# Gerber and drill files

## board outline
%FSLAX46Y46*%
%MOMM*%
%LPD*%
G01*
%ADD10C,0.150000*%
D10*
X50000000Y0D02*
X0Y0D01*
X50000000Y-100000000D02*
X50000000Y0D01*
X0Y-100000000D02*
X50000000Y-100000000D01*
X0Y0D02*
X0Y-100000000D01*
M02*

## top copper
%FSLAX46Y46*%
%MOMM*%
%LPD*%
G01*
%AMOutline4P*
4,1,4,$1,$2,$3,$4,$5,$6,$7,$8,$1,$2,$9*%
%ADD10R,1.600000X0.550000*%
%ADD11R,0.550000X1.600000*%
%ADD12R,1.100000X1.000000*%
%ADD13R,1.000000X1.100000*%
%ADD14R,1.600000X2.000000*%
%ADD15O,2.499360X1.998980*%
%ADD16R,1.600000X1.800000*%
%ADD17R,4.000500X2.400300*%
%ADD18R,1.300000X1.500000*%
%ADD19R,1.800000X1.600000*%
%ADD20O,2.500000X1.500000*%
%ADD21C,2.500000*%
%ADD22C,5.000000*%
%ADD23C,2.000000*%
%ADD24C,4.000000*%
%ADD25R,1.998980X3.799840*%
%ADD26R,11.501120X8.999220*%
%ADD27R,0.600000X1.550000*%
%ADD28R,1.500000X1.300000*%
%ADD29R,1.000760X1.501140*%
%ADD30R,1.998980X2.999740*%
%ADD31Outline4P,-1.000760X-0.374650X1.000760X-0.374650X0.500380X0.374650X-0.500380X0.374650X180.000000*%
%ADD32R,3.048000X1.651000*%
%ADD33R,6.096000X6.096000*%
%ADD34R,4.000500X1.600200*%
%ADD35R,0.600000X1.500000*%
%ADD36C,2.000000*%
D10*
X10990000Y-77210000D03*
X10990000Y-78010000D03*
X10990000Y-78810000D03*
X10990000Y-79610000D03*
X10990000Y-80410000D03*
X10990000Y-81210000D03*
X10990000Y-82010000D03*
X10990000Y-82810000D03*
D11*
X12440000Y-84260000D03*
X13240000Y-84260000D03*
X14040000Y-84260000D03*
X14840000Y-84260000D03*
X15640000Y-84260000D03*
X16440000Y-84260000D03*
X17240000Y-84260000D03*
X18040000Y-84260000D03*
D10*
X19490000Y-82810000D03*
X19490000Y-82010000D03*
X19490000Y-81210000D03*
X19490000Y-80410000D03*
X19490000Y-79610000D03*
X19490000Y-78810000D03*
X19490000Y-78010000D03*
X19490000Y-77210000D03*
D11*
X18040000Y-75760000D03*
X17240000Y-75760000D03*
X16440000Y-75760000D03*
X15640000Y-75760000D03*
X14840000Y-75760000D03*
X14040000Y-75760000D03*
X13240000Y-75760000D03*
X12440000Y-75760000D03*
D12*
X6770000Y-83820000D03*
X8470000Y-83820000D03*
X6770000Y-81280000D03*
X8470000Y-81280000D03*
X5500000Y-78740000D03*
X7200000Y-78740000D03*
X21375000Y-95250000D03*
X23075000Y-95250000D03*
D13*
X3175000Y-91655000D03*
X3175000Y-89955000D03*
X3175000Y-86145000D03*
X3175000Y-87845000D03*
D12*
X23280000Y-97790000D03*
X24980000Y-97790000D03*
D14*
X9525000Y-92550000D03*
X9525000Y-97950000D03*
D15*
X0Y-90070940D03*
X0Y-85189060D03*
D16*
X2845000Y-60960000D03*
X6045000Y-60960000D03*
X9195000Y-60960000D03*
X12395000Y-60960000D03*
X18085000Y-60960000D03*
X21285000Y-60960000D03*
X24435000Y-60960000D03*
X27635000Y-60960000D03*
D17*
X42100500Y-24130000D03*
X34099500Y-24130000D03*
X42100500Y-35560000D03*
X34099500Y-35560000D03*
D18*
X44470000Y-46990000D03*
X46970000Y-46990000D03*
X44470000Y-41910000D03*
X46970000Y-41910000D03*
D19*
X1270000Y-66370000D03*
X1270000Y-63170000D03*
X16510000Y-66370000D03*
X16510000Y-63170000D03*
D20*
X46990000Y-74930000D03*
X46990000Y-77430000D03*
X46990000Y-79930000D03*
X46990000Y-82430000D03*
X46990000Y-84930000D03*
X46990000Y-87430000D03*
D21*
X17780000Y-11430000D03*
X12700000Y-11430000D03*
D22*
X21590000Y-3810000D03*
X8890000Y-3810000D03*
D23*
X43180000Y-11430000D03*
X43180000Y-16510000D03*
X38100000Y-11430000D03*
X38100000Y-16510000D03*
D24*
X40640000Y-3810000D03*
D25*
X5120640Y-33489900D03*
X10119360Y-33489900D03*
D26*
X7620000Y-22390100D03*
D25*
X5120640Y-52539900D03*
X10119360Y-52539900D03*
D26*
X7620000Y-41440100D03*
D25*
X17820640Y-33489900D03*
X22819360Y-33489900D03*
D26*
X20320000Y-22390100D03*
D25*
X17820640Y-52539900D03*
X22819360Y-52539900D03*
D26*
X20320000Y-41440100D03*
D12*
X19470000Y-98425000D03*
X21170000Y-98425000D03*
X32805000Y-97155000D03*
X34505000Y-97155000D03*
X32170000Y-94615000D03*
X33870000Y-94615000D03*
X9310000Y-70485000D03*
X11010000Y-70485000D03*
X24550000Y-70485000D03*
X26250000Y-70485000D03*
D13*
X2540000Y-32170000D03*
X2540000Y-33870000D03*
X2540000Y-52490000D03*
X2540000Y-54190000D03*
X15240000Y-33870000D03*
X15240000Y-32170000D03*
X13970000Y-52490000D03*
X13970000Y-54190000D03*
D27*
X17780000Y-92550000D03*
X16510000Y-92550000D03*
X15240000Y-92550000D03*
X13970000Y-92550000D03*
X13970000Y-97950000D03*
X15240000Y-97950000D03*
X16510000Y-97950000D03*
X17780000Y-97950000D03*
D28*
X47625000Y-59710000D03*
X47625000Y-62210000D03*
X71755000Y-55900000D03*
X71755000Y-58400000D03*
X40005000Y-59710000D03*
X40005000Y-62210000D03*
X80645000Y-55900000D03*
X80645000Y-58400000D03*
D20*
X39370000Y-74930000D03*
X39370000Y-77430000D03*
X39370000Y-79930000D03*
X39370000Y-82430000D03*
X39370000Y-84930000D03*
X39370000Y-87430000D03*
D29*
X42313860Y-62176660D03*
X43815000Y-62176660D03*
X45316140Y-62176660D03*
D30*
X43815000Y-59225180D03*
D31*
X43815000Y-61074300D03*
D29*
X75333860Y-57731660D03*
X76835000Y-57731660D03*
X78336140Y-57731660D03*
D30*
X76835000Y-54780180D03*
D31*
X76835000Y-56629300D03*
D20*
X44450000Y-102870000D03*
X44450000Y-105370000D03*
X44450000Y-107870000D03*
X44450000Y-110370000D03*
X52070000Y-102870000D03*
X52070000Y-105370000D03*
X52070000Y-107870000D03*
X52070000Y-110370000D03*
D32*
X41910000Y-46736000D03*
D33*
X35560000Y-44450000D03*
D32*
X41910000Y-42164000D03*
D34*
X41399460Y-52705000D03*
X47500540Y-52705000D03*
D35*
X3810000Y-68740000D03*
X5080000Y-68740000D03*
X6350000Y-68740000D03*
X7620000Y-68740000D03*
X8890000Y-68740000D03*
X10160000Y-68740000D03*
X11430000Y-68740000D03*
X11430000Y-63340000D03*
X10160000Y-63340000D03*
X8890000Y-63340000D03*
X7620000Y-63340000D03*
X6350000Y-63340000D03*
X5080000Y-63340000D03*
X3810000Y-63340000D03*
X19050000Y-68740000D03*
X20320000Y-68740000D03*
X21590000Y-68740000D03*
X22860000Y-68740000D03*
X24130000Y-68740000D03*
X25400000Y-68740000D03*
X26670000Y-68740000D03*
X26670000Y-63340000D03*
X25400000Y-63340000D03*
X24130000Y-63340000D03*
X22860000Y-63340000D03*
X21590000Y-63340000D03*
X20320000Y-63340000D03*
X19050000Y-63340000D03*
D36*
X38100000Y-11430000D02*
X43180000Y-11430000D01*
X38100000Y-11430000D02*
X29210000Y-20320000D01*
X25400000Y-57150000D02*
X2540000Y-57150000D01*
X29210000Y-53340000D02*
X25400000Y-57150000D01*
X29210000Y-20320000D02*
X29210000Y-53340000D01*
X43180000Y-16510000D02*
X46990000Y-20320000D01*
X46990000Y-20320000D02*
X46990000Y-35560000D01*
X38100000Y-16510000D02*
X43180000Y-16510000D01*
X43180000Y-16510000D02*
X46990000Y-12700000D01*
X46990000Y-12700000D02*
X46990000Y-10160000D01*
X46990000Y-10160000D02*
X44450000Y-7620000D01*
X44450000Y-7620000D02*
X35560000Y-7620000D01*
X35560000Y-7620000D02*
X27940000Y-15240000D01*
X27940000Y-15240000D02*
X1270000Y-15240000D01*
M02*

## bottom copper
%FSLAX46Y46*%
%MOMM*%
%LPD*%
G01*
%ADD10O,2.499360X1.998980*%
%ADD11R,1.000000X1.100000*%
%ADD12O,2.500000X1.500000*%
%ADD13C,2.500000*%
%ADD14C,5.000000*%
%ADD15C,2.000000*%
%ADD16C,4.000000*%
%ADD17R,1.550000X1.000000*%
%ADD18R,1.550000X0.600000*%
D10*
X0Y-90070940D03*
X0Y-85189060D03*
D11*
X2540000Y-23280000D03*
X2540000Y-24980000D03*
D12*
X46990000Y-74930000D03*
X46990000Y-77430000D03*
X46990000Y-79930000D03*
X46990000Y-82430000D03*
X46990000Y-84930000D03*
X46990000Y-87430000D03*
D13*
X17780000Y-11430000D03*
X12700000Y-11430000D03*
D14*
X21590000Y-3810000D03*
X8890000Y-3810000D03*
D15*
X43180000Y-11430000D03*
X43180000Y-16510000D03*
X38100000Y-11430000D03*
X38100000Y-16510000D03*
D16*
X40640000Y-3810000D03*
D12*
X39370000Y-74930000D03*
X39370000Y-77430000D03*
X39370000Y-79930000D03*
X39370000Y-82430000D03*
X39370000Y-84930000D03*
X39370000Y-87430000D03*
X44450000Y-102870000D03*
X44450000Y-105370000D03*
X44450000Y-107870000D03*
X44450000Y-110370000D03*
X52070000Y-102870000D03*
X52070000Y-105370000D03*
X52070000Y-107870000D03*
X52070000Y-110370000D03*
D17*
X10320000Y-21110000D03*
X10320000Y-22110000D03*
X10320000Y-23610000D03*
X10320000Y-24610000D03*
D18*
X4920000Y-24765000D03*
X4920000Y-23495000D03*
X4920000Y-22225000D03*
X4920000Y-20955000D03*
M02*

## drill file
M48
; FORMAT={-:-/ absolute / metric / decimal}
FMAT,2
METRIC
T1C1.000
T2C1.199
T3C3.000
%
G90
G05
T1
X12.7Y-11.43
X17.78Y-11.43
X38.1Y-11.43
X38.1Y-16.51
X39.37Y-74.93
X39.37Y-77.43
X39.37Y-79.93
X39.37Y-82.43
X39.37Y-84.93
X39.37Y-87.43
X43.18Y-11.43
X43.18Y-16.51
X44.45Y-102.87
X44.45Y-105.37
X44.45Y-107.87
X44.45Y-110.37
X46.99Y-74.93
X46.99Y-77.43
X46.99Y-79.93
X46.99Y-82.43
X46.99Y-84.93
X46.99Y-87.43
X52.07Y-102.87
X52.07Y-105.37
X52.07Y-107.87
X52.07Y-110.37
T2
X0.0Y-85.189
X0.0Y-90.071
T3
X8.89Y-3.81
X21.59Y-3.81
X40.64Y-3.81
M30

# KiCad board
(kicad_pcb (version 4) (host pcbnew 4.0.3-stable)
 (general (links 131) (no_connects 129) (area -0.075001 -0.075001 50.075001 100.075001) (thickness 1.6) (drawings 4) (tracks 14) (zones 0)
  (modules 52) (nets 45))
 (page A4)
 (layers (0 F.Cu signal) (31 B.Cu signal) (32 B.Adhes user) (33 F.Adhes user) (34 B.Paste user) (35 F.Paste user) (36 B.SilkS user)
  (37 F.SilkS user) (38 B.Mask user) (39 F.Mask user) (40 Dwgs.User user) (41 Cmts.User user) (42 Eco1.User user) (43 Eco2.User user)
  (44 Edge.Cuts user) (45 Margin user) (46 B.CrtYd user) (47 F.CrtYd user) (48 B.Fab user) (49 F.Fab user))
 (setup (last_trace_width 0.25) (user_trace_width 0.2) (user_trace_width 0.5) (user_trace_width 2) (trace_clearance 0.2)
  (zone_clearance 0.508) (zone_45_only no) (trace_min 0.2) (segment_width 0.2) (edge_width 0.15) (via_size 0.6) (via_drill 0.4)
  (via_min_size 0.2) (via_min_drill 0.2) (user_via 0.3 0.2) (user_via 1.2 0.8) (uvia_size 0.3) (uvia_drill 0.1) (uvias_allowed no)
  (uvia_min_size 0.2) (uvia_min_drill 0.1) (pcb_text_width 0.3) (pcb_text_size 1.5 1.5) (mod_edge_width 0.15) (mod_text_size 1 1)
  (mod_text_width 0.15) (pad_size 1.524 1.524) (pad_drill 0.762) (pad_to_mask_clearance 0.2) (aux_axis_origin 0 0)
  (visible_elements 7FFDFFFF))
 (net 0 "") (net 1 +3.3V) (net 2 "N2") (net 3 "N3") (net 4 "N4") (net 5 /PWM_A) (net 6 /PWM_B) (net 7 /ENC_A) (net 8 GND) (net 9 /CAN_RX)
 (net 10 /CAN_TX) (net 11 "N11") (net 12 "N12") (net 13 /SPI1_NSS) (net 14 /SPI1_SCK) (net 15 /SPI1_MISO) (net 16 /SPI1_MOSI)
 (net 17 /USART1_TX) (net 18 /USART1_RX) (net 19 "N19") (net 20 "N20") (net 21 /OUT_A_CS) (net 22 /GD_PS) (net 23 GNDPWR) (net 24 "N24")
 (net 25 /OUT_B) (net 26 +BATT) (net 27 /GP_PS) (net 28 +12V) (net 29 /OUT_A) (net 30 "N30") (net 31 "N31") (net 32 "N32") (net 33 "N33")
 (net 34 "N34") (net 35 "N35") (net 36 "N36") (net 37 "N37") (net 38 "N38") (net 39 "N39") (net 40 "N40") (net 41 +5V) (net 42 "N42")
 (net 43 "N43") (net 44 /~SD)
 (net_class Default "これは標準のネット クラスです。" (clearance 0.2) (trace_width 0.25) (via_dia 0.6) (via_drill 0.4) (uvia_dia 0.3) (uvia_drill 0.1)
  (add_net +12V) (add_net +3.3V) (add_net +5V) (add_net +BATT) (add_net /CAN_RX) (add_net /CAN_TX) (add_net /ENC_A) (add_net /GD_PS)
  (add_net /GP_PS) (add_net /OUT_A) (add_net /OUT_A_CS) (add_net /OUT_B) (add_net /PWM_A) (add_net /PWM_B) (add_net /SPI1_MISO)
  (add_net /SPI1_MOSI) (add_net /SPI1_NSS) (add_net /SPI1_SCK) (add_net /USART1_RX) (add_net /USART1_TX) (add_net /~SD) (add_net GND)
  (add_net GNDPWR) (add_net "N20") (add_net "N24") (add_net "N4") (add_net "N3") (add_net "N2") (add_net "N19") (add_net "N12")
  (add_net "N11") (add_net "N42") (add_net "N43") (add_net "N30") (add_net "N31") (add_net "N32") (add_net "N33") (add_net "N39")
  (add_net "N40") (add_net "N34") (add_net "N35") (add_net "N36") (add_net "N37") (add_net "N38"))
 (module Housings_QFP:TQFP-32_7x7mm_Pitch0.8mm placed (layer F.Cu) (at 15.24 80.01)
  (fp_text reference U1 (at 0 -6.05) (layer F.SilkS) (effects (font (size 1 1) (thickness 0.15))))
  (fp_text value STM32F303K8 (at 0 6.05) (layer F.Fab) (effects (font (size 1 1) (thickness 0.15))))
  (pad 1 smd rect (at -4.25 -2.8) (size 1.6 0.55) (layers F.Cu F.Paste F.Mask) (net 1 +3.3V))
  (pad 2 smd rect (at -4.25 -2) (size 1.6 0.55) (layers F.Cu F.Paste F.Mask) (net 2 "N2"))
  (pad 3 smd rect (at -4.25 -1.2) (size 1.6 0.55) (layers F.Cu F.Paste F.Mask) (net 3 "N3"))
  (pad 4 smd rect (at -4.25 -0.4) (size 1.6 0.55) (layers F.Cu F.Paste F.Mask) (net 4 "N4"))
  (pad 5 smd rect (at -4.25 0.4) (size 1.6 0.55) (layers F.Cu F.Paste F.Mask) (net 1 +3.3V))
  (pad 6 smd rect (at -4.25 1.2) (size 1.6 0.55) (layers F.Cu F.Paste F.Mask) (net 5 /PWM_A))
  (pad 7 smd rect (at -4.25 2) (size 1.6 0.55) (layers F.Cu F.Paste F.Mask) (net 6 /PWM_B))
  (pad 8 smd rect (at -4.25 2.8) (size 1.6 0.55) (layers F.Cu F.Paste F.Mask))
  (pad 9 smd rect (at -2.8 4.25 90) (size 1.6 0.55) (layers F.Cu F.Paste F.Mask))
  (pad 10 smd rect (at -2 4.25 90) (size 1.6 0.55) (layers F.Cu F.Paste F.Mask))
  (pad 11 smd rect (at -1.2 4.25 90) (size 1.6 0.55) (layers F.Cu F.Paste F.Mask))
  (pad 12 smd rect (at -0.4 4.25 90) (size 1.6 0.55) (layers F.Cu F.Paste F.Mask) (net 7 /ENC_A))
  (pad 13 smd rect (at 0.4 4.25 90) (size 1.6 0.55) (layers F.Cu F.Paste F.Mask))
  (pad 14 smd rect (at 1.2 4.25 90) (size 1.6 0.55) (layers F.Cu F.Paste F.Mask))
  (pad 15 smd rect (at 2 4.25 90) (size 1.6 0.55) (layers F.Cu F.Paste F.Mask))
  (pad 16 smd rect (at 2.8 4.25 90) (size 1.6 0.55) (layers F.Cu F.Paste F.Mask) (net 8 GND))
  (pad 17 smd rect (at 4.25 2.8) (size 1.6 0.55) (layers F.Cu F.Paste F.Mask) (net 1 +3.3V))
  (pad 18 smd rect (at 4.25 2) (size 1.6 0.55) (layers F.Cu F.Paste F.Mask))
  (pad 19 smd rect (at 4.25 1.2) (size 1.6 0.55) (layers F.Cu F.Paste F.Mask))
  (pad 20 smd rect (at 4.25 0.4) (size 1.6 0.55) (layers F.Cu F.Paste F.Mask))
  (pad 21 smd rect (at 4.25 -0.4) (size 1.6 0.55) (layers F.Cu F.Paste F.Mask) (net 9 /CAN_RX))
  (pad 22 smd rect (at 4.25 -1.2) (size 1.6 0.55) (layers F.Cu F.Paste F.Mask) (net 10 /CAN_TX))
  (pad 23 smd rect (at 4.25 -2) (size 1.6 0.55) (layers F.Cu F.Paste F.Mask) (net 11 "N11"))
  (pad 24 smd rect (at 4.25 -2.8) (size 1.6 0.55) (layers F.Cu F.Paste F.Mask) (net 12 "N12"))
  (pad 25 smd rect (at 2.8 -4.25 90) (size 1.6 0.55) (layers F.Cu F.Paste F.Mask) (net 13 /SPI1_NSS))
  (pad 26 smd rect (at 2 -4.25 90) (size 1.6 0.55) (layers F.Cu F.Paste F.Mask) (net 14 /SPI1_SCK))
  (pad 27 smd rect (at 1.2 -4.25 90) (size 1.6 0.55) (layers F.Cu F.Paste F.Mask) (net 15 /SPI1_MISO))
  (pad 28 smd rect (at 0.4 -4.25 90) (size 1.6 0.55) (layers F.Cu F.Paste F.Mask) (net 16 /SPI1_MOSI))
  (pad 29 smd rect (at -0.4 -4.25 90) (size 1.6 0.55) (layers F.Cu F.Paste F.Mask) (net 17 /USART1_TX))
  (pad 30 smd rect (at -1.2 -4.25 90) (size 1.6 0.55) (layers F.Cu F.Paste F.Mask) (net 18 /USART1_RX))
  (pad 31 smd rect (at -2 -4.25 90) (size 1.6 0.55) (layers F.Cu F.Paste F.Mask) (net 8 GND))
  (pad 32 smd rect (at -2.8 -4.25 90) (size 1.6 0.55) (layers F.Cu F.Paste F.Mask) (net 8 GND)))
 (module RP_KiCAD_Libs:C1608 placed (layer F.Cu) (at 7.62 83.82)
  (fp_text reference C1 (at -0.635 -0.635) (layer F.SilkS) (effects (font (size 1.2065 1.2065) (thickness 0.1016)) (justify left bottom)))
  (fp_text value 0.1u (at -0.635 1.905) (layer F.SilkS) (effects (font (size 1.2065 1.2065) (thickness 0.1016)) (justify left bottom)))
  (pad 1 smd rect (at -0.85 0) (size 1.1 1) (layers F.Cu F.Paste F.Mask) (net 1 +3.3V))
  (pad 2 smd rect (at 0.85 0) (size 1.1 1) (layers F.Cu F.Paste F.Mask) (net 8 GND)))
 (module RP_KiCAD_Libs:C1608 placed (layer F.Cu) (at 7.62 81.28)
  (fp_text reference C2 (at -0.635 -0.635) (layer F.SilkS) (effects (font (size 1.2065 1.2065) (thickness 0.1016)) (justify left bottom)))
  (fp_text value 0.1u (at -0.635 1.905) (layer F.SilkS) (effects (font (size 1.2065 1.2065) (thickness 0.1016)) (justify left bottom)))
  (pad 1 smd rect (at -0.85 0) (size 1.1 1) (layers F.Cu F.Paste F.Mask) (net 1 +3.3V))
  (pad 2 smd rect (at 0.85 0) (size 1.1 1) (layers F.Cu F.Paste F.Mask) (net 8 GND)))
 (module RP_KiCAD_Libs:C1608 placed (layer F.Cu) (at 6.35 78.74)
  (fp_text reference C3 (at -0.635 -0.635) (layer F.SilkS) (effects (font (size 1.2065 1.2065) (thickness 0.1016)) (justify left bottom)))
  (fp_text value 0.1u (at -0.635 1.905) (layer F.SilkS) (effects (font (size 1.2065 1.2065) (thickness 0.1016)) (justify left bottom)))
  (pad 1 smd rect (at -0.85 0) (size 1.1 1) (layers F.Cu F.Paste F.Mask) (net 1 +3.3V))
  (pad 2 smd rect (at 0.85 0) (size 1.1 1) (layers F.Cu F.Paste F.Mask) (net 8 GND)))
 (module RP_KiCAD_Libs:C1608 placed (layer F.Cu) (at 22.225 95.25)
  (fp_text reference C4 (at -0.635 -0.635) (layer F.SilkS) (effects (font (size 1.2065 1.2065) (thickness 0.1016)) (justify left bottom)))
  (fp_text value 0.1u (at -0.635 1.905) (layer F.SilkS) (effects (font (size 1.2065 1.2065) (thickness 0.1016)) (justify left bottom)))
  (pad 1 smd rect (at -0.85 0) (size 1.1 1) (layers F.Cu F.Paste F.Mask) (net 8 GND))
  (pad 2 smd rect (at 0.85 0) (size 1.1 1) (layers F.Cu F.Paste F.Mask) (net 4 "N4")))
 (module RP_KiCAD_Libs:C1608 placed (layer F.Cu) (at 3.175 90.805 90)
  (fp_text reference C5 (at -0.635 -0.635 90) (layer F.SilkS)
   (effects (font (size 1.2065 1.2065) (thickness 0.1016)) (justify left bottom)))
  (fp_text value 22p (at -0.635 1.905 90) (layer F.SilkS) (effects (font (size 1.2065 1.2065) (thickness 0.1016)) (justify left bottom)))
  (pad 1 smd rect (at -0.85 0 90) (size 1.1 1) (layers F.Cu F.Paste F.Mask) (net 3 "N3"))
  (pad 2 smd rect (at 0.85 0 90) (size 1.1 1) (layers F.Cu F.Paste F.Mask) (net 8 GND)))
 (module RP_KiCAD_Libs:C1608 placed (layer F.Cu) (at 3.175 86.995 270)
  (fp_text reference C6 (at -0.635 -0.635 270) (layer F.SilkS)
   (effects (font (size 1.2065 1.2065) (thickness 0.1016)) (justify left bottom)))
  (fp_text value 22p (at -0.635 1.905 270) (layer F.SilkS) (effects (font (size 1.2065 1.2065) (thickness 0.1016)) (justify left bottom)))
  (pad 1 smd rect (at -0.85 0 270) (size 1.1 1) (layers F.Cu F.Paste F.Mask) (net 2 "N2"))
  (pad 2 smd rect (at 0.85 0 270) (size 1.1 1) (layers F.Cu F.Paste F.Mask) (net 8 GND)))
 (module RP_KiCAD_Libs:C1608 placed (layer F.Cu) (at 24.13 97.79)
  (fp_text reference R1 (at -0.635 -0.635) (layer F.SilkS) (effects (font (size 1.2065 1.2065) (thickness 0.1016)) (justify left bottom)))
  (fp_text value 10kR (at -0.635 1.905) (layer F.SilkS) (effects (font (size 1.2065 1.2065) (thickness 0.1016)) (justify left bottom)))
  (pad 1 smd rect (at -0.85 0) (size 1.1 1) (layers F.Cu F.Paste F.Mask) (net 4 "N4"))
  (pad 2 smd rect (at 0.85 0) (size 1.1 1) (layers F.Cu F.Paste F.Mask) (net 1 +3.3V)))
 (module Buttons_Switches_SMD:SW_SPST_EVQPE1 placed (layer F.Cu) (at 9.525 95.25 90)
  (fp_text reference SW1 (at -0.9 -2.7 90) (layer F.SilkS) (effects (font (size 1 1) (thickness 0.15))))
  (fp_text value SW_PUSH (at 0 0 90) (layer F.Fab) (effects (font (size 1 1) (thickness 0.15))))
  (pad 2 smd rect (at 2.7 0 90) (size 2 1.6) (layers F.Cu F.Paste F.Mask) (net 4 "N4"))
  (pad 1 smd rect (at -2.7 0 90) (size 2 1.6) (layers F.Cu F.Paste F.Mask) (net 8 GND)))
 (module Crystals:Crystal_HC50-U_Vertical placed (layer F.Cu) (at 0 87.63 90)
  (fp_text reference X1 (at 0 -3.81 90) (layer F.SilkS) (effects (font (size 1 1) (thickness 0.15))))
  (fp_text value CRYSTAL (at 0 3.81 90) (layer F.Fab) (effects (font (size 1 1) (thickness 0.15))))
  (pad 1 thru_hole oval (at -2.44094 0 90) (size 1.99898 2.49936) (drill 1.19888) (layers *.Cu *.Mask F.SilkS) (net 3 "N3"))
  (pad 2 thru_hole oval (at 2.44094 0 90) (size 1.99898 2.49936) (drill 1.19888) (layers *.Cu *.Mask F.SilkS) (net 2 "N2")))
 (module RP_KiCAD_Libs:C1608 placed (layer B.Cu) (at 2.54 24.13 270)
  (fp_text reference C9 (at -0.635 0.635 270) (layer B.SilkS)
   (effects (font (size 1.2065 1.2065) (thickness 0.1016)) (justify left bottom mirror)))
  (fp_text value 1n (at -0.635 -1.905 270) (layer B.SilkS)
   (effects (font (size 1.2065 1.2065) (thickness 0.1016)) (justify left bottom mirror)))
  (pad 1 smd rect (at -0.85 0 270) (size 1.1 1) (layers B.Cu B.Paste B.Mask) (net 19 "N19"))
  (pad 2 smd rect (at 0.85 0 270) (size 1.1 1) (layers B.Cu B.Paste B.Mask) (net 8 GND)))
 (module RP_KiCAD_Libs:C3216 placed (layer F.Cu) (at 4.445 60.96)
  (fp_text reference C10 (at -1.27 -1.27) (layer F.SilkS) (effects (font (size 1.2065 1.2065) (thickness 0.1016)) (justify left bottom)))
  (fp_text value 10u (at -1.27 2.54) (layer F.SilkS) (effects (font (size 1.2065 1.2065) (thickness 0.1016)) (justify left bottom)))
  (pad 1 smd rect (at -1.6 0) (size 1.6 1.8) (layers F.Cu F.Paste F.Mask) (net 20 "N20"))
  (pad 2 smd rect (at 1.6 0) (size 1.6 1.8) (layers F.Cu F.Paste F.Mask) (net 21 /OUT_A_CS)))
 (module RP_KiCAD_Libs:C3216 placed (layer F.Cu) (at 10.795 60.96)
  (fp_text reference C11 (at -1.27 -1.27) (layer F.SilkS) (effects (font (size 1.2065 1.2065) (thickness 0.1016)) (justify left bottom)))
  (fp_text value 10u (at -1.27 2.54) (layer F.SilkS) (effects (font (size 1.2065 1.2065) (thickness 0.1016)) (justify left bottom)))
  (pad 1 smd rect (at -1.6 0) (size 1.6 1.8) (layers F.Cu F.Paste F.Mask) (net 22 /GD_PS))
  (pad 2 smd rect (at 1.6 0) (size 1.6 1.8) (layers F.Cu F.Paste F.Mask) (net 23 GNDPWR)))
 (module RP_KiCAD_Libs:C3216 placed (layer F.Cu) (at 19.685 60.96)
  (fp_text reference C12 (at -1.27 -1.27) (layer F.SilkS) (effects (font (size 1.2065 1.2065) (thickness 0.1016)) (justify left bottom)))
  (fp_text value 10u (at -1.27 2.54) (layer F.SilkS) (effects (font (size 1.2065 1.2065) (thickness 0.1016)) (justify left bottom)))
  (pad 1 smd rect (at -1.6 0) (size 1.6 1.8) (layers F.Cu F.Paste F.Mask) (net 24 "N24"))
  (pad 2 smd rect (at 1.6 0) (size 1.6 1.8) (layers F.Cu F.Paste F.Mask) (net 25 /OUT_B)))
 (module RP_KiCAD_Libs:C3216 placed (layer F.Cu) (at 26.035 60.96)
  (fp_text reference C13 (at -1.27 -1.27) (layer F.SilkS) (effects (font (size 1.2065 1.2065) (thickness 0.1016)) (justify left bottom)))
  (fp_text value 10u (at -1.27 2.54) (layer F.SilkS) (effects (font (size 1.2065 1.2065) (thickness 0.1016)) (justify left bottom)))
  (pad 1 smd rect (at -1.6 0) (size 1.6 1.8) (layers F.Cu F.Paste F.Mask) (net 22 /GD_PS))
  (pad 2 smd rect (at 1.6 0) (size 1.6 1.8) (layers F.Cu F.Paste F.Mask) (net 23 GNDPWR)))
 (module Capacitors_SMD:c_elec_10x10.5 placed (layer F.Cu) (at 38.1 24.13)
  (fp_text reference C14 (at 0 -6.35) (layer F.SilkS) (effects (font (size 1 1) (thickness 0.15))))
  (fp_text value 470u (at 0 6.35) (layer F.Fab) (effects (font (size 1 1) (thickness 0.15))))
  (pad 1 smd rect (at 4.0005 0) (size 4.0005 2.4003) (layers F.Cu F.Paste F.Mask) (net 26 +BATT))
  (pad 2 smd rect (at -4.0005 0) (size 4.0005 2.4003) (layers F.Cu F.Paste F.Mask) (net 23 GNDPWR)))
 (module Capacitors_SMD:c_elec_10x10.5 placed (layer F.Cu) (at 38.1 35.56)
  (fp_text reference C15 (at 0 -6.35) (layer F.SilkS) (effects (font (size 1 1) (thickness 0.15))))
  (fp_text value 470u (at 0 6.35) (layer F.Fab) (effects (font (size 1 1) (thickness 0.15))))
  (pad 1 smd rect (at 4.0005 0) (size 4.0005 2.4003) (layers F.Cu F.Paste F.Mask) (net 26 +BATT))
  (pad 2 smd rect (at -4.0005 0) (size 4.0005 2.4003) (layers F.Cu F.Paste F.Mask) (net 23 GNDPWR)))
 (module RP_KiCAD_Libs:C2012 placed (layer F.Cu) (at 45.72 46.99)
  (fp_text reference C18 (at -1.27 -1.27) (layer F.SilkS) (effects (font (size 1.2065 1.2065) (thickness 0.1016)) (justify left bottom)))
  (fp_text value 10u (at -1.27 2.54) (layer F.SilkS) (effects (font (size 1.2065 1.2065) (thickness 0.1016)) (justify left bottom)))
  (pad 1 smd rect (at -1.25 0) (size 1.3 1.5) (layers F.Cu F.Paste F.Mask) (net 26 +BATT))
  (pad 2 smd rect (at 1.25 0) (size 1.3 1.5) (layers F.Cu F.Paste F.Mask) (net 23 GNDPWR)))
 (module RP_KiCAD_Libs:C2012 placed (layer F.Cu) (at 45.72 41.91)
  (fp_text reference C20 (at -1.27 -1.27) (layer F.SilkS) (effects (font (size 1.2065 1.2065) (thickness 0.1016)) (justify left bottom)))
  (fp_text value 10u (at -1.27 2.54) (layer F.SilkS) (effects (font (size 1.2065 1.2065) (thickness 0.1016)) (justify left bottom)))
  (pad 1 smd rect (at -1.25 0) (size 1.3 1.5) (layers F.Cu F.Paste F.Mask) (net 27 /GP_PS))
  (pad 2 smd rect (at 1.25 0) (size 1.3 1.5) (layers F.Cu F.Paste F.Mask) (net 23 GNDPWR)))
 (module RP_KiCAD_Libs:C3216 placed (layer F.Cu) (at 1.27 64.77 90)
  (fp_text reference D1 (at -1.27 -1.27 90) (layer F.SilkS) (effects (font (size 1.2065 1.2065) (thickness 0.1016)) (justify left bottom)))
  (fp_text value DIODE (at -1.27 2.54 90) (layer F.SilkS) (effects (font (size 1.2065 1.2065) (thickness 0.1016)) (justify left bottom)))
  (pad 1 smd rect (at -1.6 0 90) (size 1.6 1.8) (layers F.Cu F.Paste F.Mask) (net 22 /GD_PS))
  (pad 2 smd rect (at 1.6 0 90) (size 1.6 1.8) (layers F.Cu F.Paste F.Mask) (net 20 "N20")))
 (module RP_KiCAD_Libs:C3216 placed (layer F.Cu) (at 16.51 64.77 90)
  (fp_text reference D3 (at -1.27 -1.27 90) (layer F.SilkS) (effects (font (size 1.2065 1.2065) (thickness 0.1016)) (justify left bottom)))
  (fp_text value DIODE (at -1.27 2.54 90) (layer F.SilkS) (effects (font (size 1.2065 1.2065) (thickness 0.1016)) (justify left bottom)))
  (pad 1 smd rect (at -1.6 0 90) (size 1.6 1.8) (layers F.Cu F.Paste F.Mask) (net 22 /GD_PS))
  (pad 2 smd rect (at 1.6 0 90) (size 1.6 1.8) (layers F.Cu F.Paste F.Mask) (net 24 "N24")))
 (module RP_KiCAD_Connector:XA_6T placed (layer F.Cu) (at 46.99 74.93 270)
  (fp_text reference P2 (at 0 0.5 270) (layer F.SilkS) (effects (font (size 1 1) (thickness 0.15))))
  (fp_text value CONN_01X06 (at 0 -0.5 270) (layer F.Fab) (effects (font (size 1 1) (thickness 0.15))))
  (pad 6 thru_hole oval (at 0 0 270) (size 1.5 2.5) (drill 1) (layers *.Cu *.Mask F.SilkS) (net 13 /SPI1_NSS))
  (pad 5 thru_hole oval (at 2.5 0 270) (size 1.5 2.5) (drill 1) (layers *.Cu *.Mask F.SilkS) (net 14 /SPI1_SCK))
  (pad 4 thru_hole oval (at 5 0 270) (size 1.5 2.5) (drill 1) (layers *.Cu *.Mask F.SilkS) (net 15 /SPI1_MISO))
  (pad 3 thru_hole oval (at 7.5 0 270) (size 1.5 2.5) (drill 1) (layers *.Cu *.Mask F.SilkS) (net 16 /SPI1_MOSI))
  (pad 2 thru_hole oval (at 10 0 270) (size 1.5 2.5) (drill 1) (layers *.Cu *.Mask F.SilkS) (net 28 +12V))
  (pad 1 thru_hole oval (at 12.5 0 270) (size 1.5 2.5) (drill 1) (layers *.Cu *.Mask F.SilkS) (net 8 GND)))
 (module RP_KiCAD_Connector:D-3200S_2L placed (layer F.Cu) (at 17.78 11.43 180)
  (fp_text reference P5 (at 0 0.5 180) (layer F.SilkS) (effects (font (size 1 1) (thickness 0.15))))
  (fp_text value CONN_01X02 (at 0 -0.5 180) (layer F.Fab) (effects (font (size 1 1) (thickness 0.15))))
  (pad 1 thru_hole circle (at 0 0 180) (size 2.5 2.5) (drill 1) (layers *.Cu *.Mask F.SilkS) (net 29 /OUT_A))
  (pad 2 thru_hole circle (at 5.08 0 180) (size 2.5 2.5) (drill 1) (layers *.Cu *.Mask F.SilkS) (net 25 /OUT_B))
  (pad "" thru_hole circle (at -3.81 7.62 180) (size 5 5) (drill 3) (layers *.Cu *.Mask F.SilkS))
  (pad "" thru_hole circle (at 8.89 7.62 180) (size 5 5) (drill 3) (layers *.Cu *.Mask F.SilkS)))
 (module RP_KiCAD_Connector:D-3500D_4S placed (layer F.Cu) (at 40.64 11.43 180)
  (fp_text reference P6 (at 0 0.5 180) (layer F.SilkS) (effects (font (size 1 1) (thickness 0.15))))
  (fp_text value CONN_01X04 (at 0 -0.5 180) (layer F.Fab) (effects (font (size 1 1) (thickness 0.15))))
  (pad 1 thru_hole circle (at -2.54 0 180) (size 2 2) (drill 1) (layers *.Cu *.Mask F.SilkS) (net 23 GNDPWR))
  (pad 2 thru_hole circle (at -2.54 -5.08 180) (size 2 2) (drill 1) (layers *.Cu *.Mask F.SilkS) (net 26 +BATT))
  (pad 3 thru_hole circle (at 2.54 0 180) (size 2 2) (drill 1) (layers *.Cu *.Mask F.SilkS) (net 23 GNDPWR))
  (pad 4 thru_hole circle (at 2.54 -5.08 180) (size 2 2) (drill 1) (layers *.Cu *.Mask F.SilkS) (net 26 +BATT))
  (pad "" thru_hole circle (at 0 7.62 180) (size 4 4) (drill 3) (layers *.Cu *.Mask F.SilkS)))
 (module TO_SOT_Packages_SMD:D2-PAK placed (layer F.Cu) (at 7.62 27.94)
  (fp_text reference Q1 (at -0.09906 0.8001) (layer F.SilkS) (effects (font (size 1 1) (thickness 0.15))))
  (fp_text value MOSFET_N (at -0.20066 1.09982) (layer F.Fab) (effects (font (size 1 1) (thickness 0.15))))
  (pad G smd rect (at -2.49936 5.5499) (size 1.99898 3.79984) (layers F.Cu F.Paste F.Mask) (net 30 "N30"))
  (pad S smd rect (at 2.49936 5.5499) (size 1.99898 3.79984) (layers F.Cu F.Paste F.Mask) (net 21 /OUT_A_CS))
  (pad D smd rect (at 0 -5.5499) (size 11.50112 8.99922) (layers F.Cu F.Paste F.Mask) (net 26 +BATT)))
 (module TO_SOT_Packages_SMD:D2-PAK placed (layer F.Cu) (at 7.62 46.99)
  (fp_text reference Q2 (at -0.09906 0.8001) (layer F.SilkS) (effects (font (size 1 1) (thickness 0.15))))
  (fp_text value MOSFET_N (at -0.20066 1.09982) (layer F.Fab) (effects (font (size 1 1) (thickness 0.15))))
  (pad G smd rect (at -2.49936 5.5499) (size 1.99898 3.79984) (layers F.Cu F.Paste F.Mask) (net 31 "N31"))
  (pad S smd rect (at 2.49936 5.5499) (size 1.99898 3.79984) (layers F.Cu F.Paste F.Mask) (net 23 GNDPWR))
  (pad D smd rect (at 0 -5.5499) (size 11.50112 8.99922) (layers F.Cu F.Paste F.Mask) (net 21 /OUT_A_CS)))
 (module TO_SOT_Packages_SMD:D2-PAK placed (layer F.Cu) (at 20.32 27.94)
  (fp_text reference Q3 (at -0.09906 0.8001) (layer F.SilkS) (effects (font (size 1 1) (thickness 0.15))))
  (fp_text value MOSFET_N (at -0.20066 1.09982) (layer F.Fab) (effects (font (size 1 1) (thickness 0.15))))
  (pad G smd rect (at -2.49936 5.5499) (size 1.99898 3.79984) (layers F.Cu F.Paste F.Mask) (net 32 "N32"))
  (pad S smd rect (at 2.49936 5.5499) (size 1.99898 3.79984) (layers F.Cu F.Paste F.Mask) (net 25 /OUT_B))
  (pad D smd rect (at 0 -5.5499) (size 11.50112 8.99922) (layers F.Cu F.Paste F.Mask) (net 26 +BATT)))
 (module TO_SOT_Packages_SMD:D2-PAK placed (layer F.Cu) (at 20.32 46.99)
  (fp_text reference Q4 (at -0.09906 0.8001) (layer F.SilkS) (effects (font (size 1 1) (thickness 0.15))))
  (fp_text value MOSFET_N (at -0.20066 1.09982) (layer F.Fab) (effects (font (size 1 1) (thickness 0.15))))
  (pad G smd rect (at -2.49936 5.5499) (size 1.99898 3.79984) (layers F.Cu F.Paste F.Mask) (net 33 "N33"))
  (pad S smd rect (at 2.49936 5.5499) (size 1.99898 3.79984) (layers F.Cu F.Paste F.Mask) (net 23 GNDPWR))
  (pad D smd rect (at 0 -5.5499) (size 11.50112 8.99922) (layers F.Cu F.Paste F.Mask) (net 25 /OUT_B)))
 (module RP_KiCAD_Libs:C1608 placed (layer F.Cu) (at 20.32 98.425)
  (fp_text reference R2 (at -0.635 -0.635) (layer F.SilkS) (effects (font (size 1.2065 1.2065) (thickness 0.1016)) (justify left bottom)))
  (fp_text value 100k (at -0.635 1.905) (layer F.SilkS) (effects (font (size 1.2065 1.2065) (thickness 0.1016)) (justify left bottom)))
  (pad 1 smd rect (at -0.85 0) (size 1.1 1) (layers F.Cu F.Paste F.Mask) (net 8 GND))
  (pad 2 smd rect (at 0.85 0) (size 1.1 1) (layers F.Cu F.Paste F.Mask) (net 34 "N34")))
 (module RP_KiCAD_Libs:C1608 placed (layer F.Cu) (at 33.655 97.155)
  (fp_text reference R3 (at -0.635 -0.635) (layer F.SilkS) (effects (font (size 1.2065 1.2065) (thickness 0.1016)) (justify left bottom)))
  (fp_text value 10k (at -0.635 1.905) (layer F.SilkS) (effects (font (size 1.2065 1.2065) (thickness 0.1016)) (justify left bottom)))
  (pad 1 smd rect (at -0.85 0) (size 1.1 1) (layers F.Cu F.Paste F.Mask) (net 1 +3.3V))
  (pad 2 smd rect (at 0.85 0) (size 1.1 1) (layers F.Cu F.Paste F.Mask) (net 7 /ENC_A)))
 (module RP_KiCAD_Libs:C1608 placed (layer F.Cu) (at 33.02 94.615)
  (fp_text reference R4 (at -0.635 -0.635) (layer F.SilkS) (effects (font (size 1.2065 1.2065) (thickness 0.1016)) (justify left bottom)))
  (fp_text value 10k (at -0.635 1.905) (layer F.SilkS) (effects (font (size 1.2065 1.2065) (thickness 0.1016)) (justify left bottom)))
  (pad 1 smd rect (at -0.85 0) (size 1.1 1) (layers F.Cu F.Paste F.Mask) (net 1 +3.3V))
  (pad 2 smd rect (at 0.85 0) (size 1.1 1) (layers F.Cu F.Paste F.Mask) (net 7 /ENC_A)))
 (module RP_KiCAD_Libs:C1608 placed (layer F.Cu) (at 10.16 70.485)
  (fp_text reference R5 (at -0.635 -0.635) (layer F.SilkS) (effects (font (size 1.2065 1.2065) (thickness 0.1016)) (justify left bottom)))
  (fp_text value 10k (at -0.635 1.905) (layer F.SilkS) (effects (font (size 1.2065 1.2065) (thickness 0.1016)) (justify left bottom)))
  (pad 1 smd rect (at -0.85 0) (size 1.1 1) (layers F.Cu F.Paste F.Mask) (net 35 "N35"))
  (pad 2 smd rect (at 0.85 0) (size 1.1 1) (layers F.Cu F.Paste F.Mask) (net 8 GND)))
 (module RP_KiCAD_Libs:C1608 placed (layer F.Cu) (at 25.4 70.485)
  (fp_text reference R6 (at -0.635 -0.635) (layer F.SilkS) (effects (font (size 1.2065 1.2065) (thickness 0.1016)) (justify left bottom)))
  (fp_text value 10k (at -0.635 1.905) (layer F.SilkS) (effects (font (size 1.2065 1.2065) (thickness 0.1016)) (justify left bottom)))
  (pad 1 smd rect (at -0.85 0) (size 1.1 1) (layers F.Cu F.Paste F.Mask) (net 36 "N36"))
  (pad 2 smd rect (at 0.85 0) (size 1.1 1) (layers F.Cu F.Paste F.Mask) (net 8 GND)))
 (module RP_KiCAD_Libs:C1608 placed (layer F.Cu) (at 2.54 33.02 270)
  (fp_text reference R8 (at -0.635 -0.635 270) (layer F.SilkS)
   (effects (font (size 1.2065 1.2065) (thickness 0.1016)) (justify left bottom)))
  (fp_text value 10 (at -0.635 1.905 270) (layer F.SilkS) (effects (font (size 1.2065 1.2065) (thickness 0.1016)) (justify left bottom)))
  (pad 1 smd rect (at -0.85 0 270) (size 1.1 1) (layers F.Cu F.Paste F.Mask) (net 30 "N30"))
  (pad 2 smd rect (at 0.85 0 270) (size 1.1 1) (layers F.Cu F.Paste F.Mask) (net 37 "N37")))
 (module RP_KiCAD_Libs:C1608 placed (layer F.Cu) (at 2.54 53.34 270)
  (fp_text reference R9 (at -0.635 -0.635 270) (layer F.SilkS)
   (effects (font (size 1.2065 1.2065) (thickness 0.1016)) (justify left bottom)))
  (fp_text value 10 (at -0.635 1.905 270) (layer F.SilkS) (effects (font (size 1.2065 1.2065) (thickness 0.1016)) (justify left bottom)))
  (pad 1 smd rect (at -0.85 0 270) (size 1.1 1) (layers F.Cu F.Paste F.Mask) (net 31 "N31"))
  (pad 2 smd rect (at 0.85 0 270) (size 1.1 1) (layers F.Cu F.Paste F.Mask) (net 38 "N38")))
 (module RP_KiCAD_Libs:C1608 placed (layer F.Cu) (at 15.24 33.02 90)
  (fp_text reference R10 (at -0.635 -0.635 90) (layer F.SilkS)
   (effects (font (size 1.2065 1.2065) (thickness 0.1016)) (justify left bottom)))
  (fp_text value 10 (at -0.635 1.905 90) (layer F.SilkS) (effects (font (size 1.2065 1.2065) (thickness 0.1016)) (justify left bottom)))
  (pad 1 smd rect (at -0.85 0 90) (size 1.1 1) (layers F.Cu F.Paste F.Mask) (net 32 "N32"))
  (pad 2 smd rect (at 0.85 0 90) (size 1.1 1) (layers F.Cu F.Paste F.Mask) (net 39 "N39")))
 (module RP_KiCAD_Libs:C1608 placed (layer F.Cu) (at 13.97 53.34 270)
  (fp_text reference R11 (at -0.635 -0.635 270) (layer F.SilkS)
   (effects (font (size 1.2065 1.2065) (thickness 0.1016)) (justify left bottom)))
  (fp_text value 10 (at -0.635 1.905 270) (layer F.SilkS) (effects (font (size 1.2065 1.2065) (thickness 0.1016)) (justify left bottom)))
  (pad 1 smd rect (at -0.85 0 270) (size 1.1 1) (layers F.Cu F.Paste F.Mask) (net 33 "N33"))
  (pad 2 smd rect (at 0.85 0 270) (size 1.1 1) (layers F.Cu F.Paste F.Mask) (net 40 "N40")))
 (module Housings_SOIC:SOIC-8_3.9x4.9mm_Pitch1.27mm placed (layer F.Cu) (at 15.875 95.25 270)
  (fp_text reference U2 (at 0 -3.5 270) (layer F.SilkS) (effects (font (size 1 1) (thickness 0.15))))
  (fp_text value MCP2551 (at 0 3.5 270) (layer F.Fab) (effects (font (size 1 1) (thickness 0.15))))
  (pad 1 smd rect (at -2.7 -1.905 270) (size 1.55 0.6) (layers F.Cu F.Paste F.Mask) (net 10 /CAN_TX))
  (pad 2 smd rect (at -2.7 -0.635 270) (size 1.55 0.6) (layers F.Cu F.Paste F.Mask) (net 8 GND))
  (pad 3 smd rect (at -2.7 0.635 270) (size 1.55 0.6) (layers F.Cu F.Paste F.Mask) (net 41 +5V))
  (pad 4 smd rect (at -2.7 1.905 270) (size 1.55 0.6) (layers F.Cu F.Paste F.Mask) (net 9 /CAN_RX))
  (pad 5 smd rect (at 2.7 1.905 270) (size 1.55 0.6) (layers F.Cu F.Paste F.Mask))
  (pad 6 smd rect (at 2.7 0.635 270) (size 1.55 0.6) (layers F.Cu F.Paste F.Mask) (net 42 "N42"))
  (pad 7 smd rect (at 2.7 -0.635 270) (size 1.55 0.6) (layers F.Cu F.Paste F.Mask) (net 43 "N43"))
  (pad 8 smd rect (at 2.7 -1.905 270) (size 1.55 0.6) (layers F.Cu F.Paste F.Mask) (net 34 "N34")))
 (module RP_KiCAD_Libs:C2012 (layer F.Cu) (at 47.625 60.96 270)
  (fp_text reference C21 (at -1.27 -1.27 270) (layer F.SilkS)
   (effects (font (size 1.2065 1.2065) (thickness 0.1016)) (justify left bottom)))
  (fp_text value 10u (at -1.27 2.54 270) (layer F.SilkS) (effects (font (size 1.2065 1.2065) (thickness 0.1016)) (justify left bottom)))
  (pad 1 smd rect (at -1.25 0 270) (size 1.3 1.5) (layers F.Cu F.Paste F.Mask) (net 27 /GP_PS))
  (pad 2 smd rect (at 1.25 0 270) (size 1.3 1.5) (layers F.Cu F.Paste F.Mask) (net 8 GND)))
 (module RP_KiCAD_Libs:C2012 (layer F.Cu) (at 71.755 57.15 270)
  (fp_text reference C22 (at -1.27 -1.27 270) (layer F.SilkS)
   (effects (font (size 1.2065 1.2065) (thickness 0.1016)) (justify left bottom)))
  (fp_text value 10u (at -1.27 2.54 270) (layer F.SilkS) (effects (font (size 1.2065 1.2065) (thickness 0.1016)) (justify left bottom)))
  (pad 1 smd rect (at -1.25 0 270) (size 1.3 1.5) (layers F.Cu F.Paste F.Mask) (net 41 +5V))
  (pad 2 smd rect (at 1.25 0 270) (size 1.3 1.5) (layers F.Cu F.Paste F.Mask) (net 8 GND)))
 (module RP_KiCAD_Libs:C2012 (layer F.Cu) (at 40.005 60.96 270)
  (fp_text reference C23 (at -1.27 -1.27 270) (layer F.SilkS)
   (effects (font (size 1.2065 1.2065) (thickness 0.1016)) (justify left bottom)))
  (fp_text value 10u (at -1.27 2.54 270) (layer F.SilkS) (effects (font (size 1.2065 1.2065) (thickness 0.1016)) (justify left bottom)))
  (pad 1 smd rect (at -1.25 0 270) (size 1.3 1.5) (layers F.Cu F.Paste F.Mask) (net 41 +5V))
  (pad 2 smd rect (at 1.25 0 270) (size 1.3 1.5) (layers F.Cu F.Paste F.Mask) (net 8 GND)))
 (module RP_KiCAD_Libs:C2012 (layer F.Cu) (at 80.645 57.15 270)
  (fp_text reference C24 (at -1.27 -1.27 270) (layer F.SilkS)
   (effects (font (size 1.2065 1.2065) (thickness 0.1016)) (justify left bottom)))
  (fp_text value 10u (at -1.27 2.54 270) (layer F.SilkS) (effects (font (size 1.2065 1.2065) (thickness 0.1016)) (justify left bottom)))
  (pad 1 smd rect (at -1.25 0 270) (size 1.3 1.5) (layers F.Cu F.Paste F.Mask) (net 1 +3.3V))
  (pad 2 smd rect (at 1.25 0 270) (size 1.3 1.5) (layers F.Cu F.Paste F.Mask) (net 8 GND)))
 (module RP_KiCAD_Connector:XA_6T (layer F.Cu) (at 39.37 74.93 270)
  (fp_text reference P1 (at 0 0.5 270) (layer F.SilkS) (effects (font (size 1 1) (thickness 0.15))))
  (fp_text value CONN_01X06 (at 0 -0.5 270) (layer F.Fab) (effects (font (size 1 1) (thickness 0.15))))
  (pad 6 thru_hole oval (at 0 0 270) (size 1.5 2.5) (drill 1) (layers *.Cu *.Mask F.SilkS) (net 18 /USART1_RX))
  (pad 5 thru_hole oval (at 2.5 0 270) (size 1.5 2.5) (drill 1) (layers *.Cu *.Mask F.SilkS) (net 17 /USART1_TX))
  (pad 4 thru_hole oval (at 5 0 270) (size 1.5 2.5) (drill 1) (layers *.Cu *.Mask F.SilkS) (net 11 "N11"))
  (pad 3 thru_hole oval (at 7.5 0 270) (size 1.5 2.5) (drill 1) (layers *.Cu *.Mask F.SilkS) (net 12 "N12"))
  (pad 2 thru_hole oval (at 10 0 270) (size 1.5 2.5) (drill 1) (layers *.Cu *.Mask F.SilkS) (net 1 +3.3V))
  (pad 1 thru_hole oval (at 12.5 0 270) (size 1.5 2.5) (drill 1) (layers *.Cu *.Mask F.SilkS) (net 8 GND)))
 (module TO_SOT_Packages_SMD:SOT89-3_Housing (layer F.Cu) (at 43.815 60.325)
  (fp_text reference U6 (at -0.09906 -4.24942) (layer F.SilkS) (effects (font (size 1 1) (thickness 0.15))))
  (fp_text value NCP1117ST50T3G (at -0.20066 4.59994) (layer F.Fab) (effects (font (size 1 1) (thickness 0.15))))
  (pad 1 smd rect (at -1.50114 1.85166) (size 1.00076 1.50114) (layers F.Cu F.Paste F.Mask) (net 8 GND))
  (pad 2 smd rect (at 0 1.85166) (size 1.00076 1.50114) (layers F.Cu F.Paste F.Mask) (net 41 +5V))
  (pad 3 smd rect (at 1.50114 1.85166) (size 1.00076 1.50114) (layers F.Cu F.Paste F.Mask) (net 27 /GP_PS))
  (pad 2 smd rect (at 0 -1.09982) (size 1.99898 2.99974) (layers F.Cu F.Paste F.Mask) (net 41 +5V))
  (pad 2 smd trapezoid (at 0 0.7493 180) (size 1.50114 0.7493) (rect_delta 0 0.50038) (layers F.Cu F.Paste F.Mask) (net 41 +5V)))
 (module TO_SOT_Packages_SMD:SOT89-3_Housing (layer F.Cu) (at 76.835 55.88)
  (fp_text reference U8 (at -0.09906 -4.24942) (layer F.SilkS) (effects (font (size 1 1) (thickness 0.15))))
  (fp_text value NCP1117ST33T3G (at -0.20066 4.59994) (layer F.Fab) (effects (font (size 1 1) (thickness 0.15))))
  (pad 1 smd rect (at -1.50114 1.85166) (size 1.00076 1.50114) (layers F.Cu F.Paste F.Mask) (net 8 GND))
  (pad 2 smd rect (at 0 1.85166) (size 1.00076 1.50114) (layers F.Cu F.Paste F.Mask) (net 1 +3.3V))
  (pad 3 smd rect (at 1.50114 1.85166) (size 1.00076 1.50114) (layers F.Cu F.Paste F.Mask) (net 41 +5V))
  (pad 2 smd rect (at 0 -1.09982) (size 1.99898 2.99974) (layers F.Cu F.Paste F.Mask) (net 1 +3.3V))
  (pad 2 smd trapezoid (at 0 0.7493 180) (size 1.50114 0.7493) (rect_delta 0 0.50038) (layers F.Cu F.Paste F.Mask) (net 1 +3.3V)))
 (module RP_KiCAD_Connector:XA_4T (layer F.Cu) (at 44.45 102.87 270)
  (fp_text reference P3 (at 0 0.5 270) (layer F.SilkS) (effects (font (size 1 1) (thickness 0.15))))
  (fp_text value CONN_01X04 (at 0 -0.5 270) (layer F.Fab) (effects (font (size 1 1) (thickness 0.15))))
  (pad 4 thru_hole oval (at 0 0 270) (size 1.5 2.5) (drill 1) (layers *.Cu *.Mask F.SilkS) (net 7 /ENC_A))
  (pad 3 thru_hole oval (at 2.5 0 270) (size 1.5 2.5) (drill 1) (layers *.Cu *.Mask F.SilkS) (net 7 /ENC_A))
  (pad 2 thru_hole oval (at 5 0 270) (size 1.5 2.5) (drill 1) (layers *.Cu *.Mask F.SilkS) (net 41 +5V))
  (pad 1 thru_hole oval (at 7.5 0 270) (size 1.5 2.5) (drill 1) (layers *.Cu *.Mask F.SilkS) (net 8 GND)))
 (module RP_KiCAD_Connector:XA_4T (layer F.Cu) (at 52.07 102.87 270)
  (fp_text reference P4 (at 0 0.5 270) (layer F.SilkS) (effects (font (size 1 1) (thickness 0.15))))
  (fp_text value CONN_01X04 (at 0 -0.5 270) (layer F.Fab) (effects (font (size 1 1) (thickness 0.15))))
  (pad 4 thru_hole oval (at 0 0 270) (size 1.5 2.5) (drill 1) (layers *.Cu *.Mask F.SilkS) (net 43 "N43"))
  (pad 3 thru_hole oval (at 2.5 0 270) (size 1.5 2.5) (drill 1) (layers *.Cu *.Mask F.SilkS) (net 42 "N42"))
  (pad 2 thru_hole oval (at 5 0 270) (size 1.5 2.5) (drill 1) (layers *.Cu *.Mask F.SilkS) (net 28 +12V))
  (pad 1 thru_hole oval (at 7.5 0 270) (size 1.5 2.5) (drill 1) (layers *.Cu *.Mask F.SilkS) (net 8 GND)))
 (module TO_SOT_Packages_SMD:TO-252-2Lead (layer F.Cu) (at 41.91 44.45 90)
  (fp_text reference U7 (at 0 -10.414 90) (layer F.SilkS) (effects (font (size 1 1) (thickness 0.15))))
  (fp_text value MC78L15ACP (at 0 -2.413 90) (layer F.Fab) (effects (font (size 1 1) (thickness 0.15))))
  (pad 1 smd rect (at -2.286 0 90) (size 1.651 3.048) (layers F.Cu F.Paste F.Mask) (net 26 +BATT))
  (pad 2 smd rect (at 0 -6.35 90) (size 6.096 6.096) (layers F.Cu F.Paste F.Mask) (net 23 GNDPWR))
  (pad 3 smd rect (at 2.286 0 90) (size 1.651 3.048) (layers F.Cu F.Paste F.Mask) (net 27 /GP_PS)))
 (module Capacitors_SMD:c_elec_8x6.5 (layer F.Cu) (at 44.45 52.705 180)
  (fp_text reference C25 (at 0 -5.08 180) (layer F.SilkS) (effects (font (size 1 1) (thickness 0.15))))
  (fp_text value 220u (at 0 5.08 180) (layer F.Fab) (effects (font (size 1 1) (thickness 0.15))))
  (pad 1 smd rect (at 3.05054 0 180) (size 4.0005 1.6002) (layers F.Cu F.Paste F.Mask) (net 27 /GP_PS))
  (pad 2 smd rect (at -3.05054 0 180) (size 4.0005 1.6002) (layers F.Cu F.Paste F.Mask) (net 23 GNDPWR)))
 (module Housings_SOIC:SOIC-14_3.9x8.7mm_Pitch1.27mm (layer F.Cu) (at 7.62 66.04 90)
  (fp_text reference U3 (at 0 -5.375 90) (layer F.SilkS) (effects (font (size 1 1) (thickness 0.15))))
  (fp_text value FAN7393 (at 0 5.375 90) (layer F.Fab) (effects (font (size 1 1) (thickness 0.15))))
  (pad 1 smd rect (at -2.7 -3.81 90) (size 1.5 0.6) (layers F.Cu F.Paste F.Mask) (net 5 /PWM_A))
  (pad 2 smd rect (at -2.7 -2.54 90) (size 1.5 0.6) (layers F.Cu F.Paste F.Mask) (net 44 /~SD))
  (pad 3 smd rect (at -2.7 -1.27 90) (size 1.5 0.6) (layers F.Cu F.Paste F.Mask) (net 8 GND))
  (pad 4 smd rect (at -2.7 0 90) (size 1.5 0.6) (layers F.Cu F.Paste F.Mask) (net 35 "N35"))
  (pad 5 smd rect (at -2.7 1.27 90) (size 1.5 0.6) (layers F.Cu F.Paste F.Mask) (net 23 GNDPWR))
  (pad 6 smd rect (at -2.7 2.54 90) (size 1.5 0.6) (layers F.Cu F.Paste F.Mask) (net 38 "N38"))
  (pad 7 smd rect (at -2.7 3.81 90) (size 1.5 0.6) (layers F.Cu F.Paste F.Mask) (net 22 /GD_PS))
  (pad 8 smd rect (at 2.7 3.81 90) (size 1.5 0.6) (layers F.Cu F.Paste F.Mask))
  (pad 9 smd rect (at 2.7 2.54 90) (size 1.5 0.6) (layers F.Cu F.Paste F.Mask))
  (pad 10 smd rect (at 2.7 1.27 90) (size 1.5 0.6) (layers F.Cu F.Paste F.Mask))
  (pad 11 smd rect (at 2.7 0 90) (size 1.5 0.6) (layers F.Cu F.Paste F.Mask) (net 21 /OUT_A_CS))
  (pad 12 smd rect (at 2.7 -1.27 90) (size 1.5 0.6) (layers F.Cu F.Paste F.Mask) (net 37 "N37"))
  (pad 13 smd rect (at 2.7 -2.54 90) (size 1.5 0.6) (layers F.Cu F.Paste F.Mask) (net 20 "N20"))
  (pad 14 smd rect (at 2.7 -3.81 90) (size 1.5 0.6) (layers F.Cu F.Paste F.Mask)))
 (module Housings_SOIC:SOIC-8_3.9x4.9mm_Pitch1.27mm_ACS (layer B.Cu) (at 7.62 22.86 180)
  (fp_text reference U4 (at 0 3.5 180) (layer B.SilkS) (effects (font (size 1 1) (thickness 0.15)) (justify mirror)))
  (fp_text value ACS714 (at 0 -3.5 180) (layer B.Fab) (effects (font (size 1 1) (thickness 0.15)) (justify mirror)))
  (pad 1 smd rect (at -2.7 1.75 180) (size 1.55 1) (layers B.Cu B.Paste B.Mask) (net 21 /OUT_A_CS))
  (pad 2 smd rect (at -2.7 0.75 180) (size 1.55 1) (layers B.Cu B.Paste B.Mask) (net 21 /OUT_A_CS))
  (pad 3 smd rect (at -2.7 -0.75 180) (size 1.55 1) (layers B.Cu B.Paste B.Mask) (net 29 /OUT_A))
  (pad 4 smd rect (at -2.7 -1.75 180) (size 1.55 1) (layers B.Cu B.Paste B.Mask) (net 29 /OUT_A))
  (pad 5 smd rect (at 2.7 -1.905 180) (size 1.55 0.6) (layers B.Cu B.Paste B.Mask) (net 8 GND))
  (pad 6 smd rect (at 2.7 -0.635 180) (size 1.55 0.6) (layers B.Cu B.Paste B.Mask) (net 19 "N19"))
  (pad 7 smd rect (at 2.7 0.635 180) (size 1.55 0.6) (layers B.Cu B.Paste B.Mask))
  (pad 8 smd rect (at 2.7 1.905 180) (size 1.55 0.6) (layers B.Cu B.Paste B.Mask) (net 41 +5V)))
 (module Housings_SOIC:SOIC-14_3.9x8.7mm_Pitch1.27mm (layer F.Cu) (at 22.86 66.04 90)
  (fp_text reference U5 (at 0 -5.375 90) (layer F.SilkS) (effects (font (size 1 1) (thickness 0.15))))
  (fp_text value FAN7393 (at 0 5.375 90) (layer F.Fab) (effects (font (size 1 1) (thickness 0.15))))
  (pad 1 smd rect (at -2.7 -3.81 90) (size 1.5 0.6) (layers F.Cu F.Paste F.Mask) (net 6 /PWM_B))
  (pad 2 smd rect (at -2.7 -2.54 90) (size 1.5 0.6) (layers F.Cu F.Paste F.Mask) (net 44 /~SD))
  (pad 3 smd rect (at -2.7 -1.27 90) (size 1.5 0.6) (layers F.Cu F.Paste F.Mask) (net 8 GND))
  (pad 4 smd rect (at -2.7 0 90) (size 1.5 0.6) (layers F.Cu F.Paste F.Mask) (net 36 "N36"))
  (pad 5 smd rect (at -2.7 1.27 90) (size 1.5 0.6) (layers F.Cu F.Paste F.Mask) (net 23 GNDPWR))
  (pad 6 smd rect (at -2.7 2.54 90) (size 1.5 0.6) (layers F.Cu F.Paste F.Mask) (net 40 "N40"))
  (pad 7 smd rect (at -2.7 3.81 90) (size 1.5 0.6) (layers F.Cu F.Paste F.Mask) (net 22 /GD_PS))
  (pad 8 smd rect (at 2.7 3.81 90) (size 1.5 0.6) (layers F.Cu F.Paste F.Mask))
  (pad 9 smd rect (at 2.7 2.54 90) (size 1.5 0.6) (layers F.Cu F.Paste F.Mask))
  (pad 10 smd rect (at 2.7 1.27 90) (size 1.5 0.6) (layers F.Cu F.Paste F.Mask))
  (pad 11 smd rect (at 2.7 0 90) (size 1.5 0.6) (layers F.Cu F.Paste F.Mask) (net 25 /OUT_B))
  (pad 12 smd rect (at 2.7 -1.27 90) (size 1.5 0.6) (layers F.Cu F.Paste F.Mask) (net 39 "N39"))
  (pad 13 smd rect (at 2.7 -2.54 90) (size 1.5 0.6) (layers F.Cu F.Paste F.Mask) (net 24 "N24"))
  (pad 14 smd rect (at 2.7 -3.81 90) (size 1.5 0.6) (layers F.Cu F.Paste F.Mask)))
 (gr_line (start 50 0) (end 0 0) (angle 90) (layer Edge.Cuts) (width 0.15))
 (gr_line (start 50 100) (end 50 0) (angle 90) (layer Edge.Cuts) (width 0.15))
 (gr_line (start 0 100) (end 50 100) (angle 90) (layer Edge.Cuts) (width 0.15))
 (gr_line (start 0 0) (end 0 100) (angle 90) (layer Edge.Cuts) (width 0.15))
 (segment (start 38.1 11.43) (end 43.18 11.43) (width 2) (layer F.Cu) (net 23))
 (segment (start 38.1 11.43) (end 29.21 20.32) (width 2) (layer F.Cu) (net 23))
 (segment (start 25.4 57.15) (end 2.54 57.15) (width 2) (layer F.Cu) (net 23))
 (segment (start 29.21 53.34) (end 25.4 57.15) (width 2) (layer F.Cu) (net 23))
 (segment (start 29.21 20.32) (end 29.21 53.34) (width 2) (layer F.Cu) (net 23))
 (segment (start 43.18 16.51) (end 46.99 20.32) (width 2) (layer F.Cu) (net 26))
 (segment (start 46.99 20.32) (end 46.99 35.56) (width 2) (layer F.Cu) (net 26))
 (segment (start 38.1 16.51) (end 43.18 16.51) (width 2) (layer F.Cu) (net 26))
 (segment (start 43.18 16.51) (end 46.99 12.7) (width 2) (layer F.Cu) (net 26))
 (segment (start 46.99 12.7) (end 46.99 10.16) (width 2) (layer F.Cu) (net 26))
 (segment (start 46.99 10.16) (end 44.45 7.62) (width 2) (layer F.Cu) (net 26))
 (segment (start 44.45 7.62) (end 35.56 7.62) (width 2) (layer F.Cu) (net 26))
 (segment (start 35.56 7.62) (end 27.94 15.24) (width 2) (layer F.Cu) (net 26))
 (segment (start 27.94 15.24) (end 1.27 15.24) (width 2) (layer F.Cu) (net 26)))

